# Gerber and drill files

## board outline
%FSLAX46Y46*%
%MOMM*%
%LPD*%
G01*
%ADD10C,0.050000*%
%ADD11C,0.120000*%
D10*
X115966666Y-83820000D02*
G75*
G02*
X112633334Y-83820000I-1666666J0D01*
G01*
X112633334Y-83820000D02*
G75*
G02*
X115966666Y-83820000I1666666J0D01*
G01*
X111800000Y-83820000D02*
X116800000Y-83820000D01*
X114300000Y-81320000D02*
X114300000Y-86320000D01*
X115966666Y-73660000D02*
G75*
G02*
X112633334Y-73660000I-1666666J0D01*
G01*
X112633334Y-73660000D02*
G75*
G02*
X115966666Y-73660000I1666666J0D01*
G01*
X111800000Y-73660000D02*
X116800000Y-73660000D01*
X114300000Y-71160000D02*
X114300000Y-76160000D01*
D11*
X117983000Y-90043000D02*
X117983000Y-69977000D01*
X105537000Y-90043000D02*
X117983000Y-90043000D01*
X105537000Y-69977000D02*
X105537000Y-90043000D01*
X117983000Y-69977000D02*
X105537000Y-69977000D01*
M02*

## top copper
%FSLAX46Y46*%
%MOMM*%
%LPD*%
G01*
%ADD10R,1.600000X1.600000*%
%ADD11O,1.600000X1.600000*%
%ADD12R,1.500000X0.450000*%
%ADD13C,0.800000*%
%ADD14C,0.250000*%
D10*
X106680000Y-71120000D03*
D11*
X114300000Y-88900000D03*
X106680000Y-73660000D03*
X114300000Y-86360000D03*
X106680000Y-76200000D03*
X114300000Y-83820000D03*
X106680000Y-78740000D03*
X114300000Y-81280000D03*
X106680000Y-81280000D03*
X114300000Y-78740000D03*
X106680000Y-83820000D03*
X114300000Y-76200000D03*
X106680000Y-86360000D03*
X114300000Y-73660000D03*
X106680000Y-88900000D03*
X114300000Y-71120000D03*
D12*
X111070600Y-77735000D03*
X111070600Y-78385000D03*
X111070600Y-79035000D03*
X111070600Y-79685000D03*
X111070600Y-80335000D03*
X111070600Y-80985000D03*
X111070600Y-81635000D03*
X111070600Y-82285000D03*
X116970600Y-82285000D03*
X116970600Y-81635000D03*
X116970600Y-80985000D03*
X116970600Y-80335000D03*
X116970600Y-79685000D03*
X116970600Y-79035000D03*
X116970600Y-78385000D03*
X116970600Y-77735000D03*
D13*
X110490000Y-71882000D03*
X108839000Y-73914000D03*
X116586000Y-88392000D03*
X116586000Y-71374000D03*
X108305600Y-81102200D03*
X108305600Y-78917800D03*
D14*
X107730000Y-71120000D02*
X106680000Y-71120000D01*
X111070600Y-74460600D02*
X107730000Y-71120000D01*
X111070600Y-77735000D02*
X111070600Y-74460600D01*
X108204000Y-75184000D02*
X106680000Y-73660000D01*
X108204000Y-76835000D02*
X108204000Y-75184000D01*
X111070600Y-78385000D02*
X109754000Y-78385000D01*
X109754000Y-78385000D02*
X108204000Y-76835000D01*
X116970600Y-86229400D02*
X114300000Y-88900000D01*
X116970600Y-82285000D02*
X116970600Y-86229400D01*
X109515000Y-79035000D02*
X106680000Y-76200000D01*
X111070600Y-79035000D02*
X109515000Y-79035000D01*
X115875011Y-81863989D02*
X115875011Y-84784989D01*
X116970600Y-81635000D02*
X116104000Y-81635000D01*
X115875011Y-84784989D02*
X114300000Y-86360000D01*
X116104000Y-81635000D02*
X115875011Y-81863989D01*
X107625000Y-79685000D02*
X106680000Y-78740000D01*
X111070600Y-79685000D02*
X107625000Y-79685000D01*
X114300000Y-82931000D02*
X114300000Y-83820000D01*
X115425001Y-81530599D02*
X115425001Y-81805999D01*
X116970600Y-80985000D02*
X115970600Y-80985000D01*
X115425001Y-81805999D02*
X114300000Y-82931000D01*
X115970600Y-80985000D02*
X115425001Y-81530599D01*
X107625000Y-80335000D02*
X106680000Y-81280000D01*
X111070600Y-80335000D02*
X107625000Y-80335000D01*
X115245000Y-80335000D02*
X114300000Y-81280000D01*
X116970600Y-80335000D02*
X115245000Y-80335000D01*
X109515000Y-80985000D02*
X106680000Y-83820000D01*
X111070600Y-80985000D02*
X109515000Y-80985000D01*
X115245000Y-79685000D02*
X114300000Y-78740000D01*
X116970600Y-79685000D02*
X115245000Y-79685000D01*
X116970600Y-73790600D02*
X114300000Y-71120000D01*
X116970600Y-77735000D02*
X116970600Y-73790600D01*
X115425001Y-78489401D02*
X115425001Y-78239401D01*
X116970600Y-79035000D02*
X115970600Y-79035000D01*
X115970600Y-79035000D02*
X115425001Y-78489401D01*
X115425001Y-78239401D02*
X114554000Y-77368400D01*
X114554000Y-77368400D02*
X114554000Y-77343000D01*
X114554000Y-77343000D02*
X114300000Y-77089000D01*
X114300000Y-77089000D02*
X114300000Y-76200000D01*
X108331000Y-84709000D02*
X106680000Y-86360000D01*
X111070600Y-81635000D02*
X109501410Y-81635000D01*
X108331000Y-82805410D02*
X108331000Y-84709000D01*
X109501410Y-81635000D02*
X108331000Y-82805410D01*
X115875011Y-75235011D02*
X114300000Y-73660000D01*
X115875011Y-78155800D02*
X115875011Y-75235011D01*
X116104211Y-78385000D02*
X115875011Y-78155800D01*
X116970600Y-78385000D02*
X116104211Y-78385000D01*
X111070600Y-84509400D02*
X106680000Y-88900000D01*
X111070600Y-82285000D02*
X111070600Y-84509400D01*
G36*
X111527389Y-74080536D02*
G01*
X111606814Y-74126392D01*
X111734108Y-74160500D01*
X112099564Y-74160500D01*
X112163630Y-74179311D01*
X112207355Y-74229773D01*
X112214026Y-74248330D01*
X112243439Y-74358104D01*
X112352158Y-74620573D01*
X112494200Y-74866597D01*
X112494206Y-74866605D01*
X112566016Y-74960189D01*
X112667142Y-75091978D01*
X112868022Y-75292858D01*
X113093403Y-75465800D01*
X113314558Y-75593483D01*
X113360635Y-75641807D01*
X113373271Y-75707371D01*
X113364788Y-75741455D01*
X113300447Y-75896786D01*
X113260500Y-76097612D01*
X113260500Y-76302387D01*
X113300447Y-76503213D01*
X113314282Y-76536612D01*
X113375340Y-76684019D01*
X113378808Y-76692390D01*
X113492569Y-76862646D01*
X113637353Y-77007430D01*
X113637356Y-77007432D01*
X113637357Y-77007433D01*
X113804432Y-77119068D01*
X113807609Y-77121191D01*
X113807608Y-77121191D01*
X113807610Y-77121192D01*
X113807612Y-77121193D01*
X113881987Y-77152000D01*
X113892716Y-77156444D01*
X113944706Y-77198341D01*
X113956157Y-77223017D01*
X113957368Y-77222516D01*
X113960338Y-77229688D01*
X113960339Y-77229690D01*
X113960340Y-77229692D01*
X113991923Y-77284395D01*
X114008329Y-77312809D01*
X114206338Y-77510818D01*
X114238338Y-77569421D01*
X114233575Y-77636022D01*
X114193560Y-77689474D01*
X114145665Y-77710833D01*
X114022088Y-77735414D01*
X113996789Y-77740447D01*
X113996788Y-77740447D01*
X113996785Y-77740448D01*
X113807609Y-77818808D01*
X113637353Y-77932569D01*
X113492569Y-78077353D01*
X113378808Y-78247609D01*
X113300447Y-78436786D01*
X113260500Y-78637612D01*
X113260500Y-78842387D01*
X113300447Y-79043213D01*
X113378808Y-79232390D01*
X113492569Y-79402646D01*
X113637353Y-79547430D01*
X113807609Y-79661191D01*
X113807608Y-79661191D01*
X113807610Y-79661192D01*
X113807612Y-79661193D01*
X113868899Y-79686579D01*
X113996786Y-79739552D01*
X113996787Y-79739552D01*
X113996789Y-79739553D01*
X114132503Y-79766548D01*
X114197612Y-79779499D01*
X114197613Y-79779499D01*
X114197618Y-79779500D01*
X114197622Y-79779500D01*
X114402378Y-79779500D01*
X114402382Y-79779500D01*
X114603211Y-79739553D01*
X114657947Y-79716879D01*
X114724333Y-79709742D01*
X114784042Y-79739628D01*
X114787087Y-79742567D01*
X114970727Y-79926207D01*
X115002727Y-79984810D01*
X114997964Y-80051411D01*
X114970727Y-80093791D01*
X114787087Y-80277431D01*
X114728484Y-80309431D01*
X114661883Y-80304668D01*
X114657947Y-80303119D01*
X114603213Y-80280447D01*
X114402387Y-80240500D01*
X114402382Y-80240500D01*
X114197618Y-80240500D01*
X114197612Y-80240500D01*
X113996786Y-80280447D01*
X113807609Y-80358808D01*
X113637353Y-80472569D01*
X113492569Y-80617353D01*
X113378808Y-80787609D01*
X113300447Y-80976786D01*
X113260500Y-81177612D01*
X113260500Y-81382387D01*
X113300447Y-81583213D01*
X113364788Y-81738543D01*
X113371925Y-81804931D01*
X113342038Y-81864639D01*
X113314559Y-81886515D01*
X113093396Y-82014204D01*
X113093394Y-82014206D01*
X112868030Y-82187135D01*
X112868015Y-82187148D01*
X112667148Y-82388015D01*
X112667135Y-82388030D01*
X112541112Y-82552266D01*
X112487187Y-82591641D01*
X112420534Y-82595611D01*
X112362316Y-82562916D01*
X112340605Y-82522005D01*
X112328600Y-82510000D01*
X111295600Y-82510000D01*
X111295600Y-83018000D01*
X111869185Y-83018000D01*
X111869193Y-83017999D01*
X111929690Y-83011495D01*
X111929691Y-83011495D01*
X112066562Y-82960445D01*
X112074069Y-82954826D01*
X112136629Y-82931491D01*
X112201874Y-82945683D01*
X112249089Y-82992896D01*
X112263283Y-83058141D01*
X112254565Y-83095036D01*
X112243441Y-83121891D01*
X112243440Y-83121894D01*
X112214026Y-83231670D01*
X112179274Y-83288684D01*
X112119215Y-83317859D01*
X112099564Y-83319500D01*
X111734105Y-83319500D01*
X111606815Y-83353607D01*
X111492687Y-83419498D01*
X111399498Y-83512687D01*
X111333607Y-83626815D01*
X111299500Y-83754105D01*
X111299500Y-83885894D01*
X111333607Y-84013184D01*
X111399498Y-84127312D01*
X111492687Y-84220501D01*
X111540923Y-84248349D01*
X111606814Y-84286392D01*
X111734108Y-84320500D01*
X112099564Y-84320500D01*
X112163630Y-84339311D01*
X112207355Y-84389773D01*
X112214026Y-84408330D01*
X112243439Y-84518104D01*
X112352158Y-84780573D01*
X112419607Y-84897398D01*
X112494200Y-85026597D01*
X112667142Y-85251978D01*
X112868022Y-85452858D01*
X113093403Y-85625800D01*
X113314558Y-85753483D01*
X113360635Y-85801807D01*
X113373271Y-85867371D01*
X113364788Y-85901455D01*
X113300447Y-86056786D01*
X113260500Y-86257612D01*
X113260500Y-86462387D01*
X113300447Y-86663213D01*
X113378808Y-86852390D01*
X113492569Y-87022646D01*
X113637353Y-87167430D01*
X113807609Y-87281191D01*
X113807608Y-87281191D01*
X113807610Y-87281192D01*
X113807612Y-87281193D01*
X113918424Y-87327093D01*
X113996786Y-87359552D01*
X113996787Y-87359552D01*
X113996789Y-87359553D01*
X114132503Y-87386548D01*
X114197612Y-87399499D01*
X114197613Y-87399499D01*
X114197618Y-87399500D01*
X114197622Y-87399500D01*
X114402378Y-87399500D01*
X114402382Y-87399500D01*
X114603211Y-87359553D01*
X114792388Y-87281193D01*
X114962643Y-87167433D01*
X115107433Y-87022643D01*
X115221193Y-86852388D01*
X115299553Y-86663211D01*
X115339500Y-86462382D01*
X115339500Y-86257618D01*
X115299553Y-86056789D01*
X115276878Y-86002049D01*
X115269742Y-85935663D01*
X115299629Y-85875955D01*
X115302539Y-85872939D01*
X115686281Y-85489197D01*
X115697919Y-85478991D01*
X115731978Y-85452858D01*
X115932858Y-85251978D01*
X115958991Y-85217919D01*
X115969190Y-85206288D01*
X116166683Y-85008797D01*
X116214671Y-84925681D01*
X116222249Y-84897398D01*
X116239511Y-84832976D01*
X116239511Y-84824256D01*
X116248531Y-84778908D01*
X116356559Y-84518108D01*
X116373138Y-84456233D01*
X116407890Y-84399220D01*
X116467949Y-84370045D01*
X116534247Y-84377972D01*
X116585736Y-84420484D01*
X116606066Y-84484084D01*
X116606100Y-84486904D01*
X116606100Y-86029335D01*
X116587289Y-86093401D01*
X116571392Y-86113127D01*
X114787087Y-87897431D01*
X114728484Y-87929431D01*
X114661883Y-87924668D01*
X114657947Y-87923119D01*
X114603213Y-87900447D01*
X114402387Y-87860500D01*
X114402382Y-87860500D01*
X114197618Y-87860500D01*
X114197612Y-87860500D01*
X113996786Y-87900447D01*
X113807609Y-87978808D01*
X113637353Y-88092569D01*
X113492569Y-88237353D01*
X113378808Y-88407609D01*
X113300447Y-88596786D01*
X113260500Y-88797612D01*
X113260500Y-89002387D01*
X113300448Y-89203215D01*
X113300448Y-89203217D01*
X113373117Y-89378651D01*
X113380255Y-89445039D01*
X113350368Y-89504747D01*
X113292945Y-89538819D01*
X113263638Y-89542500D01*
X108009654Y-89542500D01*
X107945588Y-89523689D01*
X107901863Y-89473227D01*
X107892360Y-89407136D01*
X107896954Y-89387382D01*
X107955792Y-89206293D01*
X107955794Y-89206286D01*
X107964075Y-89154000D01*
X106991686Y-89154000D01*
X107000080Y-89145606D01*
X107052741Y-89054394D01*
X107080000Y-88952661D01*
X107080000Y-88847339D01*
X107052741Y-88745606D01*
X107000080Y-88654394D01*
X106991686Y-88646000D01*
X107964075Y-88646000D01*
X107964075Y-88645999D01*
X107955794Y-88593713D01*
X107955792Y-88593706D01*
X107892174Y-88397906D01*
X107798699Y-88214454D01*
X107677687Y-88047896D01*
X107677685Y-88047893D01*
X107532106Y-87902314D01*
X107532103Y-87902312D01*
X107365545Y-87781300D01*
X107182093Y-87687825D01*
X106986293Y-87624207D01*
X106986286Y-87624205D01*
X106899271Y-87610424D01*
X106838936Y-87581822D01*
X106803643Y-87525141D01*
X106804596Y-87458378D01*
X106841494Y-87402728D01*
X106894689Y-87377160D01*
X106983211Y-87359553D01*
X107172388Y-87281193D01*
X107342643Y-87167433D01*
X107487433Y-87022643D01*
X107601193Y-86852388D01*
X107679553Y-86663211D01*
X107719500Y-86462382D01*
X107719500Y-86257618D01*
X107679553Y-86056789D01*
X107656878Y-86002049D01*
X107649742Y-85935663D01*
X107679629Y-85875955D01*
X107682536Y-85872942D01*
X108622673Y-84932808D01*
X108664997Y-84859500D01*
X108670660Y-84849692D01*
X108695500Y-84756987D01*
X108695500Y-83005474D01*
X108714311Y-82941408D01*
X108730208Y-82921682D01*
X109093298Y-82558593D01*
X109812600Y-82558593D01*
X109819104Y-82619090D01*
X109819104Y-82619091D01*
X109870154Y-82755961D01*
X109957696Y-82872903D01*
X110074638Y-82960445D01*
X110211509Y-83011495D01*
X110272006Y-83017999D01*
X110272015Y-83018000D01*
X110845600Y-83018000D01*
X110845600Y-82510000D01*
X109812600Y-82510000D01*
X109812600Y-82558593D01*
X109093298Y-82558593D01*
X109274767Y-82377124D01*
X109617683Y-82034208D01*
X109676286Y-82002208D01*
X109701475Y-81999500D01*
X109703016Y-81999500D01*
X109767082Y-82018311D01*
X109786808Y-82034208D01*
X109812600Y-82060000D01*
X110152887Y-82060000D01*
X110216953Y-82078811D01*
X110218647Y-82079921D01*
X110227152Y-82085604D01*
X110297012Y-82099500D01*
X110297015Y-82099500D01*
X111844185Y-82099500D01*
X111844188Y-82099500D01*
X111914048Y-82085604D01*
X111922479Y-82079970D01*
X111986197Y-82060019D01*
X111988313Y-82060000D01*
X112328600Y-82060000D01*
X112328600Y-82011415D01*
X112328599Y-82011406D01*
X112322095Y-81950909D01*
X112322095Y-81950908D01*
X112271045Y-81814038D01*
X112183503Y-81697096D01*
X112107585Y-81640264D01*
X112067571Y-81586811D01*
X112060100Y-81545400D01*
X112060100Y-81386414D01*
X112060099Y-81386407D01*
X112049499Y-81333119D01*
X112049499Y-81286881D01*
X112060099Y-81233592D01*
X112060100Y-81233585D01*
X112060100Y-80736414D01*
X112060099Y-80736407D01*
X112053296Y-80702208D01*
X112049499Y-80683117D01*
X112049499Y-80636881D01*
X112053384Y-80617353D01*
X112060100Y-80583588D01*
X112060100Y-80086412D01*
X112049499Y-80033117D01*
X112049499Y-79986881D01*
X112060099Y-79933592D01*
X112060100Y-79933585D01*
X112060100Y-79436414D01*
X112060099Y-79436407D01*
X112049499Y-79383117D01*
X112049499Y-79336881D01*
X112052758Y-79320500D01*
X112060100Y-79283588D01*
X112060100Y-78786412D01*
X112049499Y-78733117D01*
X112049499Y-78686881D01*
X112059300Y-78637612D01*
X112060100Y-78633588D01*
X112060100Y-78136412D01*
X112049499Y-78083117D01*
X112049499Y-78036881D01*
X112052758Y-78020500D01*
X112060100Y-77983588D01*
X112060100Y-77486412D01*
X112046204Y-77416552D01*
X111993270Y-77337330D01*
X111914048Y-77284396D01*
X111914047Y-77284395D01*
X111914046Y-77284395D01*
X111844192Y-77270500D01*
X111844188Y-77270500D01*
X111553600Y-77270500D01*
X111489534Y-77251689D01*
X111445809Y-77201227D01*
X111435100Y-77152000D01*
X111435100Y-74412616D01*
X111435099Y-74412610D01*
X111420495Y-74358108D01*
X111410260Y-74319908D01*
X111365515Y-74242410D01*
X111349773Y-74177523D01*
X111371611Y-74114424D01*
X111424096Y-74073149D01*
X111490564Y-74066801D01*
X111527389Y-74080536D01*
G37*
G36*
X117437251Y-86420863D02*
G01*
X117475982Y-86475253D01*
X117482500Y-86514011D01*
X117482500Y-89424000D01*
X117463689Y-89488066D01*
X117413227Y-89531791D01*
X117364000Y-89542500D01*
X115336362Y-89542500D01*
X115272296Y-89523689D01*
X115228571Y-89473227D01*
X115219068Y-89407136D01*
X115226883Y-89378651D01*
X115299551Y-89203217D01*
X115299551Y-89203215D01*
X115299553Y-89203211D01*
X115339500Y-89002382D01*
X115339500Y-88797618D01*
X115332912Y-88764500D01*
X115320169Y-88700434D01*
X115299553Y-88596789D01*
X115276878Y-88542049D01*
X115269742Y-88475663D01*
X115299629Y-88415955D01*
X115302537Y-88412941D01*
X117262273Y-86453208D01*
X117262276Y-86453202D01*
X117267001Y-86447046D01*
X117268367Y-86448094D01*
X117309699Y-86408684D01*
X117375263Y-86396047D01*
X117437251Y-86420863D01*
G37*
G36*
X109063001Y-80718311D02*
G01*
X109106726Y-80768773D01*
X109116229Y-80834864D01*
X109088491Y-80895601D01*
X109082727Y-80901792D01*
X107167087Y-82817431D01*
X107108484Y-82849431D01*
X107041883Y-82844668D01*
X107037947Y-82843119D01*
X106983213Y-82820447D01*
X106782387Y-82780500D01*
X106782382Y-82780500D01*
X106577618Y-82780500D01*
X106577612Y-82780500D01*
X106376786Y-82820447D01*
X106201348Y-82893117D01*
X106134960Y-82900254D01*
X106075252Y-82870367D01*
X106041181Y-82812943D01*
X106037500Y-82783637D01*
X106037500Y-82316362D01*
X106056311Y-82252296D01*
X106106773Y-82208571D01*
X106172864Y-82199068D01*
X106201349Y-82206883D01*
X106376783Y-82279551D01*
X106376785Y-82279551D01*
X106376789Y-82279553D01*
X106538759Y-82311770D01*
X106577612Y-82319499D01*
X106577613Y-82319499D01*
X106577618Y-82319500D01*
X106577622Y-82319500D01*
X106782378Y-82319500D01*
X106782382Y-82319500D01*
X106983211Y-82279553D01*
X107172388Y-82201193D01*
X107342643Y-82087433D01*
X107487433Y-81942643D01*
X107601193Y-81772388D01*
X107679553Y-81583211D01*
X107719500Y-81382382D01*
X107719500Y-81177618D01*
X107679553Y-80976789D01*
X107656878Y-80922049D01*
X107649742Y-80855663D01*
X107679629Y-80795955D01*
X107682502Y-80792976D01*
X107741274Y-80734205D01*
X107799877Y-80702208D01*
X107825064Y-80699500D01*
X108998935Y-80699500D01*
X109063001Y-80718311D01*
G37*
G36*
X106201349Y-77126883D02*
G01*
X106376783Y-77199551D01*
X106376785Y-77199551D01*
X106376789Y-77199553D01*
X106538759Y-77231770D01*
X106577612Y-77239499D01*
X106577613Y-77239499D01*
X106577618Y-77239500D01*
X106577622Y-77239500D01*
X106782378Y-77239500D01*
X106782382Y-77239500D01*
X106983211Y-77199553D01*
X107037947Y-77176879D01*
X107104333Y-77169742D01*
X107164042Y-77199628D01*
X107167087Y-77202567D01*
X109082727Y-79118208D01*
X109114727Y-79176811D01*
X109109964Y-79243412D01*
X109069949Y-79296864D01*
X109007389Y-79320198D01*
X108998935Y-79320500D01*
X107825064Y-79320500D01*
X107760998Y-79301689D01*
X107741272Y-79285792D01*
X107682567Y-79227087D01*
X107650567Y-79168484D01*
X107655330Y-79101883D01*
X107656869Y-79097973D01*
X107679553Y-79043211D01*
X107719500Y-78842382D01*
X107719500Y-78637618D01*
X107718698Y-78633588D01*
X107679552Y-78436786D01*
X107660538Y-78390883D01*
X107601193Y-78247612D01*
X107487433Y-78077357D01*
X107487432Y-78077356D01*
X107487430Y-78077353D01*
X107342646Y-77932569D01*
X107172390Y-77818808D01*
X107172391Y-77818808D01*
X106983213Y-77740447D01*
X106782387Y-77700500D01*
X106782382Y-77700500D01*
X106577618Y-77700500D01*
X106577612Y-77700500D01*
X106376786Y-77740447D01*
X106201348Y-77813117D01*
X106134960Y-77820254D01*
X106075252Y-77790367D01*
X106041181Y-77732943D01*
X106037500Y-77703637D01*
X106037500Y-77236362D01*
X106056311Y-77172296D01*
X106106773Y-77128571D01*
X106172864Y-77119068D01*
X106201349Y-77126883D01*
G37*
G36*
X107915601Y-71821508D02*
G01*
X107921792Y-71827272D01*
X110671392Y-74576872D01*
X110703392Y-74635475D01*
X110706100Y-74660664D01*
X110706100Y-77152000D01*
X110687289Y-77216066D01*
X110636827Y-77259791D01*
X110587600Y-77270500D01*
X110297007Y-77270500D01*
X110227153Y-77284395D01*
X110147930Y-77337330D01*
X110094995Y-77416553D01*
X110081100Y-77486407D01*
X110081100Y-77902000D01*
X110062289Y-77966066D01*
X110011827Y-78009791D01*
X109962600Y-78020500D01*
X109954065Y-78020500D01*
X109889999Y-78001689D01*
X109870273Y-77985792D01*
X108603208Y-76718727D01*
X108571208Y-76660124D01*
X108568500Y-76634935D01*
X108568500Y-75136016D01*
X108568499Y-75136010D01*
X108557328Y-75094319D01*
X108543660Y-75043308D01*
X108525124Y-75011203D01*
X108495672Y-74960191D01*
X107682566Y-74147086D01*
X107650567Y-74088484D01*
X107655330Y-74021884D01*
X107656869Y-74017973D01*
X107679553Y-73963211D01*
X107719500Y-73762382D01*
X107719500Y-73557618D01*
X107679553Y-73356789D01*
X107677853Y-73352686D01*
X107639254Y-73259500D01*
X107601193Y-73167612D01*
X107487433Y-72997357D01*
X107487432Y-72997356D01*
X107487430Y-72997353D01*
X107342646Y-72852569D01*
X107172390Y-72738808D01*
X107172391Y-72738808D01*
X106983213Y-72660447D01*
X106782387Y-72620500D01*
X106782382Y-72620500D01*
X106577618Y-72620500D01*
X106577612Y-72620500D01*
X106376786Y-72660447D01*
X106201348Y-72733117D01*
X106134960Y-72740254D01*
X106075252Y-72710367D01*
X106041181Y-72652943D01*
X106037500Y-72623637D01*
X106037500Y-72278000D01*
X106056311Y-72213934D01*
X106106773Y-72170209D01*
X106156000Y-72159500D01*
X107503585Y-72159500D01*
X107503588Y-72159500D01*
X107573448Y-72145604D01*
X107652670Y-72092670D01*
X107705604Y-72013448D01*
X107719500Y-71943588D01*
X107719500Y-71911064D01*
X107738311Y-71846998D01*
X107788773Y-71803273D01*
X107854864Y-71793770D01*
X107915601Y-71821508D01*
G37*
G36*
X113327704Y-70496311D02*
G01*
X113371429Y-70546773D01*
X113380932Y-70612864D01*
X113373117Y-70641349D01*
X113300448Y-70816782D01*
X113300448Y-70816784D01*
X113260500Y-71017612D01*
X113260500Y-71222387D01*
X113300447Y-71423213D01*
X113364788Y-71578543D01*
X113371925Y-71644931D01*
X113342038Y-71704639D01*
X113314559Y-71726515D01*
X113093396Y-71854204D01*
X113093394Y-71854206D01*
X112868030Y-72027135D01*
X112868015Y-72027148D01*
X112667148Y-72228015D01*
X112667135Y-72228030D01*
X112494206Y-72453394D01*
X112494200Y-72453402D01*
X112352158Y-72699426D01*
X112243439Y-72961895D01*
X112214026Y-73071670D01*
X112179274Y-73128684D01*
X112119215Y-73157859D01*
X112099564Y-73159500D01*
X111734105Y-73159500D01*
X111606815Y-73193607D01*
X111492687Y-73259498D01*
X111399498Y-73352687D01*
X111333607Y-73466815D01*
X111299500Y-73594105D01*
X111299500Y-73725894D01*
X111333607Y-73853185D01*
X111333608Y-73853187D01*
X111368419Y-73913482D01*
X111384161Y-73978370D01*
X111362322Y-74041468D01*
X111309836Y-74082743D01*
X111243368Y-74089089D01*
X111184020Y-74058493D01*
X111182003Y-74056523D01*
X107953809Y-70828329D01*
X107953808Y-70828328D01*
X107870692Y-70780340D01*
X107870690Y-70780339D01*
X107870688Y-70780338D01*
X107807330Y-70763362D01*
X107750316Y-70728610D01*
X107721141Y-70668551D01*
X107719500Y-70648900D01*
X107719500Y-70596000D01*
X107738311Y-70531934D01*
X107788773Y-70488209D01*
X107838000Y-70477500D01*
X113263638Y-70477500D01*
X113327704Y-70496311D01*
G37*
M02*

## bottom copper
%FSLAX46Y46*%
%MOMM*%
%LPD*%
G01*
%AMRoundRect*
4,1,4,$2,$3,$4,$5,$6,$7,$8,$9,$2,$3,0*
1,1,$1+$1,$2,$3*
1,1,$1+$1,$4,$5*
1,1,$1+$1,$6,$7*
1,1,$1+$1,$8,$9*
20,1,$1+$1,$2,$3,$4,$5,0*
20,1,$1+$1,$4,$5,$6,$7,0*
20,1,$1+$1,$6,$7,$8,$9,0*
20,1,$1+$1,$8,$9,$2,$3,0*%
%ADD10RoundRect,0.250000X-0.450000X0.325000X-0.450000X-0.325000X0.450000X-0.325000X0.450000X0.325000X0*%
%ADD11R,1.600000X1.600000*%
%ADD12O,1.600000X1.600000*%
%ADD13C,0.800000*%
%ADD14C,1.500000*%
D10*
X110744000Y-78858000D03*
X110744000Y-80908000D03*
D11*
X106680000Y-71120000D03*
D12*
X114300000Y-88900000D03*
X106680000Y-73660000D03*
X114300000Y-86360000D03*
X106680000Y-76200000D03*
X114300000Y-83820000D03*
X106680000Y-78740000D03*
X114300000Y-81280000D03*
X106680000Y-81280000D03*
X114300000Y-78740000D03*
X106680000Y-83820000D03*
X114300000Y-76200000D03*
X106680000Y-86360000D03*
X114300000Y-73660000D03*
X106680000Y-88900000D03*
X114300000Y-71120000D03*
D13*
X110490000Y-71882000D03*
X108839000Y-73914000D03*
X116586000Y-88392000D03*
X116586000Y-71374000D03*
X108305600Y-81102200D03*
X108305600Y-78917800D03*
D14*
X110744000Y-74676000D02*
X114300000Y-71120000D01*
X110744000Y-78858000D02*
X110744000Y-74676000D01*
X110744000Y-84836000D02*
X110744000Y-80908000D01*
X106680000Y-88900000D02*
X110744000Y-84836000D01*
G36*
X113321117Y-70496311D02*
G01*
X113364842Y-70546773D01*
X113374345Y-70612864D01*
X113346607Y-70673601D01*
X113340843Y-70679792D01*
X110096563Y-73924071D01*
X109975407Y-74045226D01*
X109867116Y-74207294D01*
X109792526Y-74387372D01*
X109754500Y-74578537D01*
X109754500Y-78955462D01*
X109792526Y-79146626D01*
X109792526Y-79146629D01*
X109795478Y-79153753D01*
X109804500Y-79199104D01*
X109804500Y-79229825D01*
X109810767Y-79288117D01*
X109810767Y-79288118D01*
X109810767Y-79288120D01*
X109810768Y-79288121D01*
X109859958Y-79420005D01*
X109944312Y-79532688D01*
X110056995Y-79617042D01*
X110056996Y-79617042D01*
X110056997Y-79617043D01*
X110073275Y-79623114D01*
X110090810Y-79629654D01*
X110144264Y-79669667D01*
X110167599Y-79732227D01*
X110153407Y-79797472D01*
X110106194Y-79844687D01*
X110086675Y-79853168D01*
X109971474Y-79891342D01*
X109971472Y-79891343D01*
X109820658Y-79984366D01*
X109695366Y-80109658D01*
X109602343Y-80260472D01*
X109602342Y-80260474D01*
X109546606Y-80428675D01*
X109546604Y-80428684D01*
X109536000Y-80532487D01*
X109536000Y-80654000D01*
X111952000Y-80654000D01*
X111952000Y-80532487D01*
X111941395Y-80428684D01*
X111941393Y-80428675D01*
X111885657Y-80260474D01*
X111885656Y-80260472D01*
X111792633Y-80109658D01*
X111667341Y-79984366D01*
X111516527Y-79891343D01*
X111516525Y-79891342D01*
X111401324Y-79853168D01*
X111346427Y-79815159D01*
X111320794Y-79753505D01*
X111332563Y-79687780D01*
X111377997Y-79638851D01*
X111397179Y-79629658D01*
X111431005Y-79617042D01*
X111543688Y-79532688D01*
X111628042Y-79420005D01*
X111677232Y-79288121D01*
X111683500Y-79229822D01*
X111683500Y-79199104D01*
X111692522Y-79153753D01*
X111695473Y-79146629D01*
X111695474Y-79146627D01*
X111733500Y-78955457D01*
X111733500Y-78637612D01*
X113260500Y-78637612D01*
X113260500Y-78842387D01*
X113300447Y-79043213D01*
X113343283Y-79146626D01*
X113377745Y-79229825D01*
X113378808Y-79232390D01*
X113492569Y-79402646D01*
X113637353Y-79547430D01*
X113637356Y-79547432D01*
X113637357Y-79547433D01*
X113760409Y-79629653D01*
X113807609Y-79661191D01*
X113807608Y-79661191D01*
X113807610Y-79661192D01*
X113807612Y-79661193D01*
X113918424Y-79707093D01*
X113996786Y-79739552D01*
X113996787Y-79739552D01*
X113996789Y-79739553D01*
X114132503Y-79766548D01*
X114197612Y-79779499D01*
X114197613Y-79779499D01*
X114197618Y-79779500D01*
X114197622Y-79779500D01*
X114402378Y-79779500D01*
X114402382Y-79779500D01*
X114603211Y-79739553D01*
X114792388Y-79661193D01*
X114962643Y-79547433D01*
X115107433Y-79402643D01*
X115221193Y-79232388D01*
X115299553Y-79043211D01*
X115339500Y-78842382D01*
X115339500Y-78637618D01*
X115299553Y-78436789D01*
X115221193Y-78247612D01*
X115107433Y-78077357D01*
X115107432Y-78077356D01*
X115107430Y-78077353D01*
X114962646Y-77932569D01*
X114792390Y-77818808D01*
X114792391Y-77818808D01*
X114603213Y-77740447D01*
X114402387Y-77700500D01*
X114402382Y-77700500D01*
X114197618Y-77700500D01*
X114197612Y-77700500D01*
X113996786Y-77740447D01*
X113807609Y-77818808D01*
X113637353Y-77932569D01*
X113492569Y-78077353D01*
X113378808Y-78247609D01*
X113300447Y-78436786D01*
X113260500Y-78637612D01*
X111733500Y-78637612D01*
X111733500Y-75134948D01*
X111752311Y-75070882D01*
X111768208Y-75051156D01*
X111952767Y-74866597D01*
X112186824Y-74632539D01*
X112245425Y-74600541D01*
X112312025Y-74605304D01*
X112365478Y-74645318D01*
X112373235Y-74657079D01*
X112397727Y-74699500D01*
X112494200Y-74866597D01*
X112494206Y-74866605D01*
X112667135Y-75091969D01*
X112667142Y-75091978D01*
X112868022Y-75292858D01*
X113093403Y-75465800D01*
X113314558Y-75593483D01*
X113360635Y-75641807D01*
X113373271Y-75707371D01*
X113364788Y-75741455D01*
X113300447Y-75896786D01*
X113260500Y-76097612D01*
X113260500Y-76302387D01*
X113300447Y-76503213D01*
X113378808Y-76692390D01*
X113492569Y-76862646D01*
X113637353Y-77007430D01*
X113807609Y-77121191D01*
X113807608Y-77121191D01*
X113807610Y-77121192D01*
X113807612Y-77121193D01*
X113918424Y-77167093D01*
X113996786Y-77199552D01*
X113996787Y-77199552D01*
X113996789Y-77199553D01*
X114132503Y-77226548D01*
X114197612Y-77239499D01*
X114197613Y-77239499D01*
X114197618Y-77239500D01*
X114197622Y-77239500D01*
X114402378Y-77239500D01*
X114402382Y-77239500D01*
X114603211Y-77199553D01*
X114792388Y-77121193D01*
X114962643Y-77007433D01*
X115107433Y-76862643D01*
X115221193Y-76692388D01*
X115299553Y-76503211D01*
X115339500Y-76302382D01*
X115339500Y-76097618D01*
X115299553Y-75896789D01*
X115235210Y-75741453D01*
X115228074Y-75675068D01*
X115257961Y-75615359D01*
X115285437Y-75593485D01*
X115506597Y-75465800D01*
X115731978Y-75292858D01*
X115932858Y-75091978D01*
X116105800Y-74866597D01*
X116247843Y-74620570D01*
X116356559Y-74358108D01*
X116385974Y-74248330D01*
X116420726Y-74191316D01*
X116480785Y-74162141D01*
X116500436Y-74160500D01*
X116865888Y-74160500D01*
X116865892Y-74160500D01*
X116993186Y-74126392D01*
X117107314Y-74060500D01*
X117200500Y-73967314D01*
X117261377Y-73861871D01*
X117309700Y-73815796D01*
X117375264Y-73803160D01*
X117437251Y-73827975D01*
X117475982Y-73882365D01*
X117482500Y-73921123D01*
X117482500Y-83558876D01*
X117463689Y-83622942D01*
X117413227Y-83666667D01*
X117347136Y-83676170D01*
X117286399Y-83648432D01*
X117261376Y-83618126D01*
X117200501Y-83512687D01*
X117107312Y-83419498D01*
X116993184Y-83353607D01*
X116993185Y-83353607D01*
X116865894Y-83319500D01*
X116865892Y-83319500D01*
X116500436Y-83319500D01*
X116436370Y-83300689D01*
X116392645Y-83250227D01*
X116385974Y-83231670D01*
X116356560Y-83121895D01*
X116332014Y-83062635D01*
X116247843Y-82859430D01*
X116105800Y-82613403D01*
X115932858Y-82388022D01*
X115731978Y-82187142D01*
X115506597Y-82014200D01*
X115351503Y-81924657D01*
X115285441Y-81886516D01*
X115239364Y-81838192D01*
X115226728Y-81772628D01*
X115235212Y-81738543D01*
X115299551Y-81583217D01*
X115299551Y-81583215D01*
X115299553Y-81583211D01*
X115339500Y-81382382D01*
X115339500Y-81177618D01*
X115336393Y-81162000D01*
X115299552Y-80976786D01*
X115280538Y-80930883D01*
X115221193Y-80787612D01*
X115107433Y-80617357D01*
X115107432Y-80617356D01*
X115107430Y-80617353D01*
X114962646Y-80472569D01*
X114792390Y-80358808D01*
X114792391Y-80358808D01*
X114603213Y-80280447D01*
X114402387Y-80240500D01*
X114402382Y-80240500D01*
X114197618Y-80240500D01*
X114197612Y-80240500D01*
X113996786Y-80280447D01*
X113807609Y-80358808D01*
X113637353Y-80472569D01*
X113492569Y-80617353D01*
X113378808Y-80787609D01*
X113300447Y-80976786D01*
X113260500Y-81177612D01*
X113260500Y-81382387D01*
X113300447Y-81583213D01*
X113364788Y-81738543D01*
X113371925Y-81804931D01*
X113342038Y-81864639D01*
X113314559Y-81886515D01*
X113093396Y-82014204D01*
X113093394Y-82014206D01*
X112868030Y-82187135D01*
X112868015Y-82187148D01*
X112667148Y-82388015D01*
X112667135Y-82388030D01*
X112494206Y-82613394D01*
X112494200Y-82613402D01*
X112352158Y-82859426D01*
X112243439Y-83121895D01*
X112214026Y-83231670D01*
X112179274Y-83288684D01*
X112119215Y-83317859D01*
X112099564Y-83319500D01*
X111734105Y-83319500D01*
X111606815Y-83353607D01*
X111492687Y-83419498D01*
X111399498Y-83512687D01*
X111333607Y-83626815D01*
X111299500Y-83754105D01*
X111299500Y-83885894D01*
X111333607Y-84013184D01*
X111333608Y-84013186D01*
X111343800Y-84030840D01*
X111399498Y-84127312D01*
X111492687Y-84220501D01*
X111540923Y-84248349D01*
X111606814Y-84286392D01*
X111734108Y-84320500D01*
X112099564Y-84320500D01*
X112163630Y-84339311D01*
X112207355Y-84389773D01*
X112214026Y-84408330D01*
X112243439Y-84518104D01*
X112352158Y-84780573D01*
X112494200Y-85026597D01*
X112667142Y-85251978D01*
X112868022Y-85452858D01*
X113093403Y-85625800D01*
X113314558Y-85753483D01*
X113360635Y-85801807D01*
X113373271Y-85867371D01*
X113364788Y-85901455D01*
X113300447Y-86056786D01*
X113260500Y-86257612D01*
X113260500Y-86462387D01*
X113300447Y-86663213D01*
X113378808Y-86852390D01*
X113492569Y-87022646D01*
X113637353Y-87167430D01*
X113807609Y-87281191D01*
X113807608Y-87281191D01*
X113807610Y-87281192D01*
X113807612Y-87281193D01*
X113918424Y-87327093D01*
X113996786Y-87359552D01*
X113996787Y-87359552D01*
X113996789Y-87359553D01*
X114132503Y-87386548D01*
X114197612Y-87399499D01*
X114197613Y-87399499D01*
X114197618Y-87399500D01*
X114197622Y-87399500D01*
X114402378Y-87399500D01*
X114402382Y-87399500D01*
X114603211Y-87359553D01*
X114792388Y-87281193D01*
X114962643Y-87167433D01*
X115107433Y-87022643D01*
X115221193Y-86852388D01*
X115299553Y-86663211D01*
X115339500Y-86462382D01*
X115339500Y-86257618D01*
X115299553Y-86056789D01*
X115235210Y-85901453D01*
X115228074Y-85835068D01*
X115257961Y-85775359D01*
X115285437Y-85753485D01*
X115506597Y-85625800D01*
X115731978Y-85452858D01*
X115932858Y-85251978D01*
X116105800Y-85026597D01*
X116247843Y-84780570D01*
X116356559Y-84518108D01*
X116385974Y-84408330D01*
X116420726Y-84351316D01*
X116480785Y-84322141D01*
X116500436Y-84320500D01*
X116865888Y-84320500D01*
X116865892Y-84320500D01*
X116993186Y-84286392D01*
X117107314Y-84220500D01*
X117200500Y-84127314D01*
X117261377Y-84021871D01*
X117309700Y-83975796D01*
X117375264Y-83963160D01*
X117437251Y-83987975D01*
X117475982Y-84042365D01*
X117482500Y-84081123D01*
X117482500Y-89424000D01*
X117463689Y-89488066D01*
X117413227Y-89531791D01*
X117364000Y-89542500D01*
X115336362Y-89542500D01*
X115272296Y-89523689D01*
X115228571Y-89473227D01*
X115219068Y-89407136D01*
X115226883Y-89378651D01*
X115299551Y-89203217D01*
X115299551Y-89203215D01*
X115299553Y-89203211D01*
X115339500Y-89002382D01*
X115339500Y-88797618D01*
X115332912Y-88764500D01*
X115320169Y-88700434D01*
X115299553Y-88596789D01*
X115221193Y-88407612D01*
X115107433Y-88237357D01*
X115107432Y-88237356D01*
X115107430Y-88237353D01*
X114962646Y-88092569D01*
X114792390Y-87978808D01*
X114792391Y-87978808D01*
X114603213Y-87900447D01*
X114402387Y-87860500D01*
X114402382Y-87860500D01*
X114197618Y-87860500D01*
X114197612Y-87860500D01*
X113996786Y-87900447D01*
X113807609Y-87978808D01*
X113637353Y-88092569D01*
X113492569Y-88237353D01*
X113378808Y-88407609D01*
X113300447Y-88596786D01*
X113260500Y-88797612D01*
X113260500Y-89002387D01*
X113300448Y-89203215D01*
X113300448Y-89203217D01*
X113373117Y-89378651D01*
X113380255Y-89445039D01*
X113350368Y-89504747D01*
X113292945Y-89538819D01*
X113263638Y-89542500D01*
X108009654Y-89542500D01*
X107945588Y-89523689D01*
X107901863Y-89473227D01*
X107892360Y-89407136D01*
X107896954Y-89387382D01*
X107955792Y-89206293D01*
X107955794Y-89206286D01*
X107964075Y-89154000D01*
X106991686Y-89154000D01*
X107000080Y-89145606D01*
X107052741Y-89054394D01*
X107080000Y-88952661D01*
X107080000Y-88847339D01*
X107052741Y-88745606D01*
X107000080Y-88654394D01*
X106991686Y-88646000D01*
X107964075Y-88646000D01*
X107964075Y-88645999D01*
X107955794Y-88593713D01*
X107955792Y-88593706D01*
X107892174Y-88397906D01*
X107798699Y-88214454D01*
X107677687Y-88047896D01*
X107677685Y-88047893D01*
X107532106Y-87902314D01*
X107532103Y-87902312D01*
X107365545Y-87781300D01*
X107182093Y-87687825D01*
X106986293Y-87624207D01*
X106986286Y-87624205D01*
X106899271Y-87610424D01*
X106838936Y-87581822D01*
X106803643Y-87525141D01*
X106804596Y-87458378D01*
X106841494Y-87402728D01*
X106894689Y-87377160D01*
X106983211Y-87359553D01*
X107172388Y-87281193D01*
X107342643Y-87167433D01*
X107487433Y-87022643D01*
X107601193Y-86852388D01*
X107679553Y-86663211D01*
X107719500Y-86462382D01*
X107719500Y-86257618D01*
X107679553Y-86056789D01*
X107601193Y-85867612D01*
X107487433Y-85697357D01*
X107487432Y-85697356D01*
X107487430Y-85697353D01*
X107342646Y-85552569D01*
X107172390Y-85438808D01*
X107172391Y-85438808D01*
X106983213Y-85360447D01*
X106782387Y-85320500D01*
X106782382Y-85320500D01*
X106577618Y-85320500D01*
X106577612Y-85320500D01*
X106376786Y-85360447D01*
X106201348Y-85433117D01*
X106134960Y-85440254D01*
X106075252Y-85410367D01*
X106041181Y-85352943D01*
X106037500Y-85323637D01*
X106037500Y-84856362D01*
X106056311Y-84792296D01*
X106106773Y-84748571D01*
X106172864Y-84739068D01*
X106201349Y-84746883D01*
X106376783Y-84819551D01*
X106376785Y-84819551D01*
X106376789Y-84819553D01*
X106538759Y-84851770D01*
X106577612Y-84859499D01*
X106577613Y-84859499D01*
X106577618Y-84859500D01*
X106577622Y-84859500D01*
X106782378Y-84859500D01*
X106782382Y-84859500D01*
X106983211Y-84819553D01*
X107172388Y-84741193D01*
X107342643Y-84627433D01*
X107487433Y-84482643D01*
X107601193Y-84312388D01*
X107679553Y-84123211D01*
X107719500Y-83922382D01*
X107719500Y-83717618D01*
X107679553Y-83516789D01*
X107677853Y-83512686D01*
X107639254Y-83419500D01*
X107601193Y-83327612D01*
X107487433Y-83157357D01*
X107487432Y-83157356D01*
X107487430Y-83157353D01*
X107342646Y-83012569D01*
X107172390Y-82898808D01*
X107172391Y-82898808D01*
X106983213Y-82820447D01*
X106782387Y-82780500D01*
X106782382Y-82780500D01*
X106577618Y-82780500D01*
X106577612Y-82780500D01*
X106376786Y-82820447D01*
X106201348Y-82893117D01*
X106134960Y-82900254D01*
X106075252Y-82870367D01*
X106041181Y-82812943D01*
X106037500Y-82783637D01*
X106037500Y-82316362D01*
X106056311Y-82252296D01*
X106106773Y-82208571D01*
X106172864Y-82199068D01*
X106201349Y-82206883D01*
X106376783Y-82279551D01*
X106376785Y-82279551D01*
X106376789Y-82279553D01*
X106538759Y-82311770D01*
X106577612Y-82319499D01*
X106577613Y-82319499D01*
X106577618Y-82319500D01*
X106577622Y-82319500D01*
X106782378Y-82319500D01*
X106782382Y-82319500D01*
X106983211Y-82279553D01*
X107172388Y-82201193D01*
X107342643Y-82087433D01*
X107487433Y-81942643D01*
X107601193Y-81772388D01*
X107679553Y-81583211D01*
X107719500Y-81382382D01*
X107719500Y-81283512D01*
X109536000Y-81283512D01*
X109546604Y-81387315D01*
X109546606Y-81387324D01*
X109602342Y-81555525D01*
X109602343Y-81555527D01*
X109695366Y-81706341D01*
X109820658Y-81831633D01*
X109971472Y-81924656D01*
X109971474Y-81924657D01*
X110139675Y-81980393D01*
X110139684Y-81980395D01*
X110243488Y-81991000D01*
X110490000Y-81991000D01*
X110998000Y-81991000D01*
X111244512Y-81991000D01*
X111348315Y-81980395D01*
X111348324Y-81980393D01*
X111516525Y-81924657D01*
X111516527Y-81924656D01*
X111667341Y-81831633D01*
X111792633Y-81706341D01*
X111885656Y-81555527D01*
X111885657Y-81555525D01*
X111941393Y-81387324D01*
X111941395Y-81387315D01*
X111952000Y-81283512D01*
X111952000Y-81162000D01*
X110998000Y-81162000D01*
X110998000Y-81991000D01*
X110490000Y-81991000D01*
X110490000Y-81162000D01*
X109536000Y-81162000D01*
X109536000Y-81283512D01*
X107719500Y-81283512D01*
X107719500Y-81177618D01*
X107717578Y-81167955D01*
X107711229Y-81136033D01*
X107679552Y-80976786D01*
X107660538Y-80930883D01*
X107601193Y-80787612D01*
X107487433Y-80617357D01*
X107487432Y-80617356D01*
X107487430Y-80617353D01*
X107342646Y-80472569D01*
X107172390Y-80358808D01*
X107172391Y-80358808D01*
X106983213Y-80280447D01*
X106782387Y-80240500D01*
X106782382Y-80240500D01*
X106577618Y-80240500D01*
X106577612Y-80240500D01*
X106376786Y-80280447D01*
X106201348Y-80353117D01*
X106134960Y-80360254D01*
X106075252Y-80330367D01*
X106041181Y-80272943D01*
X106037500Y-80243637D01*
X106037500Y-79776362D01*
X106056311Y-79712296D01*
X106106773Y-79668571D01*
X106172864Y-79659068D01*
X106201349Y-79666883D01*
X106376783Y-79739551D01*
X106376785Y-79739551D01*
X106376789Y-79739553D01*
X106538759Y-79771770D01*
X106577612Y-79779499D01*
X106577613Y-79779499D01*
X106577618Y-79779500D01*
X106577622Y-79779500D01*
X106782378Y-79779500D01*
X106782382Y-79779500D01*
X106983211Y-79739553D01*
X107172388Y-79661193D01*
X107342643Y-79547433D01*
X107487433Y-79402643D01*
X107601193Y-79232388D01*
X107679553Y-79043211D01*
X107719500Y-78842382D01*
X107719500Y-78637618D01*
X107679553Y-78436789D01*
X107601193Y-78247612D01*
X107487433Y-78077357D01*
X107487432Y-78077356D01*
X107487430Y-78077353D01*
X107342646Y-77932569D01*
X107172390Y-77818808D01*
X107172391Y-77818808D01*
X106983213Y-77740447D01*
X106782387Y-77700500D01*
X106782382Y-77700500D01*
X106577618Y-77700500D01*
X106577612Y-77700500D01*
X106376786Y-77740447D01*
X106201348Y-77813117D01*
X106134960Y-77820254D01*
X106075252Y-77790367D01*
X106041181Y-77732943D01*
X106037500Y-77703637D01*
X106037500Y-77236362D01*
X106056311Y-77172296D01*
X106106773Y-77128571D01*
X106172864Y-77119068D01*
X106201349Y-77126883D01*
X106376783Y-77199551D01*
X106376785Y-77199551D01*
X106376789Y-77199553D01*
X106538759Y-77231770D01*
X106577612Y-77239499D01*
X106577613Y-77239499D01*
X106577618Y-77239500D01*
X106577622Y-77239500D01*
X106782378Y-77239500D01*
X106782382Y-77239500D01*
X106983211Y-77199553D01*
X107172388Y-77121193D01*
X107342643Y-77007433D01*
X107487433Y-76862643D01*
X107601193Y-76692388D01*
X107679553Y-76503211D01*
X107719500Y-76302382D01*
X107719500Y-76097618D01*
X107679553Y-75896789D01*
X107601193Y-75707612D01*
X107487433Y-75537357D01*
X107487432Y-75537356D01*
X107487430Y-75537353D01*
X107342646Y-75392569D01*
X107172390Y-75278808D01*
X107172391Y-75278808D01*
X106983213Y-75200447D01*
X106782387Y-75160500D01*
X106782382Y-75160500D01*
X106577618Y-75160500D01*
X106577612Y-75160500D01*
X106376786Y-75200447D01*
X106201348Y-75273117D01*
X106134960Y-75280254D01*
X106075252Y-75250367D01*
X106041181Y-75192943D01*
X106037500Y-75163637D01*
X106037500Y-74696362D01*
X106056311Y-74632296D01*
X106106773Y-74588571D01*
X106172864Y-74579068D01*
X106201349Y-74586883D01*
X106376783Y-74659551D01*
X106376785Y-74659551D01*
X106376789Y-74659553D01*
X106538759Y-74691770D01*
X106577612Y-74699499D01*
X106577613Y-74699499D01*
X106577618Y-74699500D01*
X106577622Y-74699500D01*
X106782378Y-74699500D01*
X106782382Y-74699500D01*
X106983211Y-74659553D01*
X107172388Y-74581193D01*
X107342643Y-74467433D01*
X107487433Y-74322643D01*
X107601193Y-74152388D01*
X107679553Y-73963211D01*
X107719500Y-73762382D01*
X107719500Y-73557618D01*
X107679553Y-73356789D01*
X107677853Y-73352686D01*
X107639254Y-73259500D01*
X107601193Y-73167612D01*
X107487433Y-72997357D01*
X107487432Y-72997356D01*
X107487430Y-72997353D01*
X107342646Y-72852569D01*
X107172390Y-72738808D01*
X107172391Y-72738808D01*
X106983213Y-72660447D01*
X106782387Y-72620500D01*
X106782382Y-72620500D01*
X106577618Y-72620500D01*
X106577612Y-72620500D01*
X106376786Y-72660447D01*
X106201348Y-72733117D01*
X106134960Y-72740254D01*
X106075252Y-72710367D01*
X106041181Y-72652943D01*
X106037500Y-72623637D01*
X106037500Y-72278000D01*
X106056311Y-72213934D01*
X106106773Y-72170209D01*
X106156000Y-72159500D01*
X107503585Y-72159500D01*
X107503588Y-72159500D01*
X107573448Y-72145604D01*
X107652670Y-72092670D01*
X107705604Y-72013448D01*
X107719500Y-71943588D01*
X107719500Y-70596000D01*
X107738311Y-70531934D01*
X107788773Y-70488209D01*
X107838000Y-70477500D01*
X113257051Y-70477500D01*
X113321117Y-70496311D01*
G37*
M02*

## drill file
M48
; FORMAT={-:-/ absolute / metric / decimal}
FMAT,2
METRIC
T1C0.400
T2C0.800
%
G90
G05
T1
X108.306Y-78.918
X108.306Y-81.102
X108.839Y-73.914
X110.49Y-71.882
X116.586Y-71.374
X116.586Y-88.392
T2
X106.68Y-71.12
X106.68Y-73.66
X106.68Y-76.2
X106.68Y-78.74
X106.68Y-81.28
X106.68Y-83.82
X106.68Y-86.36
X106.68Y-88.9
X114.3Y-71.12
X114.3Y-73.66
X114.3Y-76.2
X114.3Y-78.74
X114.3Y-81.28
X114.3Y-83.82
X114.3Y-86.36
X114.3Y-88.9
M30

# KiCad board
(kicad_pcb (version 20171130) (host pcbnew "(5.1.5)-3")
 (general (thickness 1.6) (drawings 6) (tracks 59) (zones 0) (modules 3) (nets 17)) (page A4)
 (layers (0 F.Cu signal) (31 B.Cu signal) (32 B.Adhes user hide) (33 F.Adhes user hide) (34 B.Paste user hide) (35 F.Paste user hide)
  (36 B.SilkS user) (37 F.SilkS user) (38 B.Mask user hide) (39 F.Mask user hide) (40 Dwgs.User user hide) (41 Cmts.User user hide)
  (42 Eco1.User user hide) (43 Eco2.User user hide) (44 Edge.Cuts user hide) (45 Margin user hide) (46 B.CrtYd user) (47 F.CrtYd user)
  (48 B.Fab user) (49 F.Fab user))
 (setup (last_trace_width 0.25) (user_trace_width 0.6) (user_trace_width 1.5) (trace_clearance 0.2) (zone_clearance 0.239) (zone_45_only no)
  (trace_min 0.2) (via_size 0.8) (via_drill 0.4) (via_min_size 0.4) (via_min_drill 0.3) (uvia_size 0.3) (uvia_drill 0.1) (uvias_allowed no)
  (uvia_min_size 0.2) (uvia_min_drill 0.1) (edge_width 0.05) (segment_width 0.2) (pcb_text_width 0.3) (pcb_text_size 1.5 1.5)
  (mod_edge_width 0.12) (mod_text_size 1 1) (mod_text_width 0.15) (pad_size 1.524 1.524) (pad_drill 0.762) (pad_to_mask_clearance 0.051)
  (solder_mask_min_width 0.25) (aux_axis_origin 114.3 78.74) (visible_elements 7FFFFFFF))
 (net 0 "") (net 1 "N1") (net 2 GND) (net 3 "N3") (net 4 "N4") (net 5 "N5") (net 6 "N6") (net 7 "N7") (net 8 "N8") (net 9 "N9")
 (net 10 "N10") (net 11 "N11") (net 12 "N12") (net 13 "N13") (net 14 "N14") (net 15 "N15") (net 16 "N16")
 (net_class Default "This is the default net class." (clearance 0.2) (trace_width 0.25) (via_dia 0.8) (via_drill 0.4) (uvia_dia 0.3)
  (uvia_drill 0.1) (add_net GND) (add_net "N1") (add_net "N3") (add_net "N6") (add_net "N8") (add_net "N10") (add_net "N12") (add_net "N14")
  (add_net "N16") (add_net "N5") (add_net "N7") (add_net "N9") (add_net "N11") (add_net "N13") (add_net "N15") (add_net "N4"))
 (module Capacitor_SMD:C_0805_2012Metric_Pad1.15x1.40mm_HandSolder (layer B.Cu) (at 110.744 79.883 270)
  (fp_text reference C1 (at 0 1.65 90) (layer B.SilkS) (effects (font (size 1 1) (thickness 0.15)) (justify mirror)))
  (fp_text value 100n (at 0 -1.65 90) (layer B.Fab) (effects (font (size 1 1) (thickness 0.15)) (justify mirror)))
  (pad 1 smd roundrect (at -1.025 0 270) (size 1.15 1.4) (layers B.Cu B.Paste B.Mask) (roundrect_rratio 0.217391) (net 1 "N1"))
  (pad 2 smd roundrect (at 1.025 0 270) (size 1.15 1.4) (layers B.Cu B.Paste B.Mask) (roundrect_rratio 0.217391) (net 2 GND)))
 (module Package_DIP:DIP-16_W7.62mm (layer F.Cu) (at 106.68 71.12)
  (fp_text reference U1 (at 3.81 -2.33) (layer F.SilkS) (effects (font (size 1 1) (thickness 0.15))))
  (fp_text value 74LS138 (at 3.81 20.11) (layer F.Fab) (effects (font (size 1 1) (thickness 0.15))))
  (pad 1 thru_hole rect (at 0 0) (size 1.6 1.6) (drill 0.8) (layers *.Cu *.Mask) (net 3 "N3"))
  (pad 9 thru_hole oval (at 7.62 17.78) (size 1.6 1.6) (drill 0.8) (layers *.Cu *.Mask) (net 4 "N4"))
  (pad 2 thru_hole oval (at 0 2.54) (size 1.6 1.6) (drill 0.8) (layers *.Cu *.Mask) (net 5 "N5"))
  (pad 10 thru_hole oval (at 7.62 15.24) (size 1.6 1.6) (drill 0.8) (layers *.Cu *.Mask) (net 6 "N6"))
  (pad 3 thru_hole oval (at 0 5.08) (size 1.6 1.6) (drill 0.8) (layers *.Cu *.Mask) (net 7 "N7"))
  (pad 11 thru_hole oval (at 7.62 12.7) (size 1.6 1.6) (drill 0.8) (layers *.Cu *.Mask) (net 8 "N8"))
  (pad 4 thru_hole oval (at 0 7.62) (size 1.6 1.6) (drill 0.8) (layers *.Cu *.Mask) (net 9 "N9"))
  (pad 12 thru_hole oval (at 7.62 10.16) (size 1.6 1.6) (drill 0.8) (layers *.Cu *.Mask) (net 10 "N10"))
  (pad 5 thru_hole oval (at 0 10.16) (size 1.6 1.6) (drill 0.8) (layers *.Cu *.Mask) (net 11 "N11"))
  (pad 13 thru_hole oval (at 7.62 7.62) (size 1.6 1.6) (drill 0.8) (layers *.Cu *.Mask) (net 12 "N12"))
  (pad 6 thru_hole oval (at 0 12.7) (size 1.6 1.6) (drill 0.8) (layers *.Cu *.Mask) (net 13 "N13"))
  (pad 14 thru_hole oval (at 7.62 5.08) (size 1.6 1.6) (drill 0.8) (layers *.Cu *.Mask) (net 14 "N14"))
  (pad 7 thru_hole oval (at 0 15.24) (size 1.6 1.6) (drill 0.8) (layers *.Cu *.Mask) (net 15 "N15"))
  (pad 15 thru_hole oval (at 7.62 2.54) (size 1.6 1.6) (drill 0.8) (layers *.Cu *.Mask) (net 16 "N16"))
  (pad 8 thru_hole oval (at 0 17.78) (size 1.6 1.6) (drill 0.8) (layers *.Cu *.Mask) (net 2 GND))
  (pad 16 thru_hole oval (at 7.62 0) (size 1.6 1.6) (drill 0.8) (layers *.Cu *.Mask) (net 1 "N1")))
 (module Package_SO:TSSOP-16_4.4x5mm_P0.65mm (layer F.Cu) (at 114.0206 80.01)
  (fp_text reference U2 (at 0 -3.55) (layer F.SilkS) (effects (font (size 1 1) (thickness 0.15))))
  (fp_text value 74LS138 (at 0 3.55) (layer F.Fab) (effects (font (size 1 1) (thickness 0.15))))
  (pad 1 smd rect (at -2.95 -2.275) (size 1.5 0.45) (layers F.Cu F.Paste F.Mask) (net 3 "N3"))
  (pad 2 smd rect (at -2.95 -1.625) (size 1.5 0.45) (layers F.Cu F.Paste F.Mask) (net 5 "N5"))
  (pad 3 smd rect (at -2.95 -0.975) (size 1.5 0.45) (layers F.Cu F.Paste F.Mask) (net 7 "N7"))
  (pad 4 smd rect (at -2.95 -0.325) (size 1.5 0.45) (layers F.Cu F.Paste F.Mask) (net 9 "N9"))
  (pad 5 smd rect (at -2.95 0.325) (size 1.5 0.45) (layers F.Cu F.Paste F.Mask) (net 11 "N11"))
  (pad 6 smd rect (at -2.95 0.975) (size 1.5 0.45) (layers F.Cu F.Paste F.Mask) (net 13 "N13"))
  (pad 7 smd rect (at -2.95 1.625) (size 1.5 0.45) (layers F.Cu F.Paste F.Mask) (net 15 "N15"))
  (pad 8 smd rect (at -2.95 2.275) (size 1.5 0.45) (layers F.Cu F.Paste F.Mask) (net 2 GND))
  (pad 9 smd rect (at 2.95 2.275) (size 1.5 0.45) (layers F.Cu F.Paste F.Mask) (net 4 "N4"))
  (pad 10 smd rect (at 2.95 1.625) (size 1.5 0.45) (layers F.Cu F.Paste F.Mask) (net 6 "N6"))
  (pad 11 smd rect (at 2.95 0.975) (size 1.5 0.45) (layers F.Cu F.Paste F.Mask) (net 8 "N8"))
  (pad 12 smd rect (at 2.95 0.325) (size 1.5 0.45) (layers F.Cu F.Paste F.Mask) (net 10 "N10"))
  (pad 13 smd rect (at 2.95 -0.325) (size 1.5 0.45) (layers F.Cu F.Paste F.Mask) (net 12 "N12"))
  (pad 14 smd rect (at 2.95 -0.975) (size 1.5 0.45) (layers F.Cu F.Paste F.Mask) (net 14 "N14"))
  (pad 15 smd rect (at 2.95 -1.625) (size 1.5 0.45) (layers F.Cu F.Paste F.Mask) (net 16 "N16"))
  (pad 16 smd rect (at 2.95 -2.275) (size 1.5 0.45) (layers F.Cu F.Paste F.Mask) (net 1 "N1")))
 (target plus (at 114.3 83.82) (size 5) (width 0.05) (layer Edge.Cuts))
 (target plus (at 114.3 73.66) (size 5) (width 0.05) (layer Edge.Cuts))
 (gr_line (start 117.983 90.043) (end 117.983 69.977) (layer Edge.Cuts) (width 0.12))
 (gr_line (start 105.537 90.043) (end 117.983 90.043) (layer Edge.Cuts) (width 0.12))
 (gr_line (start 105.537 69.977) (end 105.537 90.043) (layer Edge.Cuts) (width 0.12))
 (gr_line (start 117.983 69.977) (end 105.537 69.977) (layer Edge.Cuts) (width 0.12))
 (segment (start 107.73 71.12) (end 106.68 71.12) (width 0.25) (layer F.Cu) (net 3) (status 20))
 (segment (start 111.0706 74.4606) (end 107.73 71.12) (width 0.25) (layer F.Cu) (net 3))
 (segment (start 111.0706 77.735) (end 111.0706 74.4606) (width 0.25) (layer F.Cu) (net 3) (status 10))
 (segment (start 108.204 75.184) (end 106.68 73.66) (width 0.25) (layer F.Cu) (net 5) (status 20))
 (segment (start 108.204 76.835) (end 108.204 75.184) (width 0.25) (layer F.Cu) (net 5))
 (segment (start 111.0706 78.385) (end 109.754 78.385) (width 0.25) (layer F.Cu) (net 5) (status 10))
 (segment (start 109.754 78.385) (end 108.204 76.835) (width 0.25) (layer F.Cu) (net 5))
 (segment (start 116.9706 86.2294) (end 114.3 88.9) (width 0.25) (layer F.Cu) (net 4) (status 20))
 (segment (start 116.9706 82.285) (end 116.9706 86.2294) (width 0.25) (layer F.Cu) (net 4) (status 10))
 (segment (start 109.515 79.035) (end 106.68 76.2) (width 0.25) (layer F.Cu) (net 7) (status 20))
 (segment (start 111.0706 79.035) (end 109.515 79.035) (width 0.25) (layer F.Cu) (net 7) (status 10))
 (segment (start 115.875011 81.863989) (end 115.875011 84.784989) (width 0.25) (layer F.Cu) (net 6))
 (segment (start 116.9706 81.635) (end 116.104 81.635) (width 0.25) (layer F.Cu) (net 6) (status 10))
 (segment (start 115.875011 84.784989) (end 114.3 86.36) (width 0.25) (layer F.Cu) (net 6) (status 20))
 (segment (start 116.104 81.635) (end 115.875011 81.863989) (width 0.25) (layer F.Cu) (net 6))
 (segment (start 107.625 79.685) (end 106.68 78.74) (width 0.25) (layer F.Cu) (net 9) (status 20))
 (segment (start 111.0706 79.685) (end 107.625 79.685) (width 0.25) (layer F.Cu) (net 9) (status 10))
 (segment (start 114.3 82.931) (end 114.3 83.82) (width 0.25) (layer F.Cu) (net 8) (status 20))
 (segment (start 115.425001 81.530599) (end 115.425001 81.805999) (width 0.25) (layer F.Cu) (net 8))
 (segment (start 116.9706 80.985) (end 115.9706 80.985) (width 0.25) (layer F.Cu) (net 8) (status 10))
 (segment (start 115.425001 81.805999) (end 114.3 82.931) (width 0.25) (layer F.Cu) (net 8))
 (segment (start 115.9706 80.985) (end 115.425001 81.530599) (width 0.25) (layer F.Cu) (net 8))
 (segment (start 107.625 80.335) (end 106.68 81.28) (width 0.25) (layer F.Cu) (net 11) (status 20))
 (segment (start 111.0706 80.335) (end 107.625 80.335) (width 0.25) (layer F.Cu) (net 11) (status 10))
 (segment (start 115.245 80.335) (end 114.3 81.28) (width 0.25) (layer F.Cu) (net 10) (status 20))
 (segment (start 116.9706 80.335) (end 115.245 80.335) (width 0.25) (layer F.Cu) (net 10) (status 10))
 (segment (start 109.515 80.985) (end 106.68 83.82) (width 0.25) (layer F.Cu) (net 13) (status 20))
 (segment (start 111.0706 80.985) (end 109.515 80.985) (width 0.25) (layer F.Cu) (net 13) (status 10))
 (segment (start 115.245 79.685) (end 114.3 78.74) (width 0.25) (layer F.Cu) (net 12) (status 20))
 (segment (start 116.9706 79.685) (end 115.245 79.685) (width 0.25) (layer F.Cu) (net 12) (status 10))
 (segment (start 116.9706 73.7906) (end 114.3 71.12) (width 0.25) (layer F.Cu) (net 1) (status 20))
 (segment (start 116.9706 77.735) (end 116.9706 73.7906) (width 0.25) (layer F.Cu) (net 1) (status 10))
 (segment (start 110.744 74.676) (end 114.3 71.12) (width 1.5) (layer B.Cu) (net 1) (status 20))
 (segment (start 110.744 78.858) (end 110.744 74.676) (width 1.5) (layer B.Cu) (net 1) (status 10))
 (segment (start 115.425001 78.489401) (end 115.425001 78.239401) (width 0.25) (layer F.Cu) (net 14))
 (segment (start 116.9706 79.035) (end 115.9706 79.035) (width 0.25) (layer F.Cu) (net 14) (status 10))
 (segment (start 115.9706 79.035) (end 115.425001 78.489401) (width 0.25) (layer F.Cu) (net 14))
 (segment (start 115.425001 78.239401) (end 114.554 77.3684) (width 0.25) (layer F.Cu) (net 14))
 (segment (start 114.554 77.3684) (end 114.554 77.343) (width 0.25) (layer F.Cu) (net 14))
 (segment (start 114.554 77.343) (end 114.3 77.089) (width 0.25) (layer F.Cu) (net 14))
 (segment (start 114.3 77.089) (end 114.3 76.2) (width 0.25) (layer F.Cu) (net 14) (status 20))
 (segment (start 108.331 84.709) (end 106.68 86.36) (width 0.25) (layer F.Cu) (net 15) (status 20))
 (segment (start 111.0706 81.635) (end 109.50141 81.635) (width 0.25) (layer F.Cu) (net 15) (status 10))
 (segment (start 108.331 82.80541) (end 108.331 84.709) (width 0.25) (layer F.Cu) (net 15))
 (segment (start 109.50141 81.635) (end 108.331 82.80541) (width 0.25) (layer F.Cu) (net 15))
 (segment (start 115.875011 75.235011) (end 114.3 73.66) (width 0.25) (layer F.Cu) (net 16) (status 20))
 (segment (start 115.875011 78.1558) (end 115.875011 75.235011) (width 0.25) (layer F.Cu) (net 16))
 (segment (start 116.104211 78.385) (end 115.875011 78.1558) (width 0.25) (layer F.Cu) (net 16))
 (segment (start 116.9706 78.385) (end 116.104211 78.385) (width 0.25) (layer F.Cu) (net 16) (status 10))
 (segment (start 111.0706 84.5094) (end 106.68 88.9) (width 0.25) (layer F.Cu) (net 2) (status 20))
 (segment (start 111.0706 82.285) (end 111.0706 84.5094) (width 0.25) (layer F.Cu) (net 2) (status 10))
 (segment (start 110.744 84.836) (end 110.744 80.908) (width 1.5) (layer B.Cu) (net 2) (status 20))
 (segment (start 106.68 88.9) (end 110.744 84.836) (width 1.5) (layer B.Cu) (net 2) (status 10))
 (via (at 110.49 71.882) (size 0.8) (drill 0.4) (layers F.Cu B.Cu) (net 2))
 (via (at 108.839 73.914) (size 0.8) (drill 0.4) (layers F.Cu B.Cu) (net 2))
 (via (at 116.586 88.392) (size 0.8) (drill 0.4) (layers F.Cu B.Cu) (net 2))
 (via (at 116.586 71.374) (size 0.8) (drill 0.4) (layers F.Cu B.Cu) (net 2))
 (via (at 108.3056 81.1022) (size 0.8) (drill 0.4) (layers F.Cu B.Cu) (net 2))
 (via (at 108.3056 78.9178) (size 0.8) (drill 0.4) (layers F.Cu B.Cu) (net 2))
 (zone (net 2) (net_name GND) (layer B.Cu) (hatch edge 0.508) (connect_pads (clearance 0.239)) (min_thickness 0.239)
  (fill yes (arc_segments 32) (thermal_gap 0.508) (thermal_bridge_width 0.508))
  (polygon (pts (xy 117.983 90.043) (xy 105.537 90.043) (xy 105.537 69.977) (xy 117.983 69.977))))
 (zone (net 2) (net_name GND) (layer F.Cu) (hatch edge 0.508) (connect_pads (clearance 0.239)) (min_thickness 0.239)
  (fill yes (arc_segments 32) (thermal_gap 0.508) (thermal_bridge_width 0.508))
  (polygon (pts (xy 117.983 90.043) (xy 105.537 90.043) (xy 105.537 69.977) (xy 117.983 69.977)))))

